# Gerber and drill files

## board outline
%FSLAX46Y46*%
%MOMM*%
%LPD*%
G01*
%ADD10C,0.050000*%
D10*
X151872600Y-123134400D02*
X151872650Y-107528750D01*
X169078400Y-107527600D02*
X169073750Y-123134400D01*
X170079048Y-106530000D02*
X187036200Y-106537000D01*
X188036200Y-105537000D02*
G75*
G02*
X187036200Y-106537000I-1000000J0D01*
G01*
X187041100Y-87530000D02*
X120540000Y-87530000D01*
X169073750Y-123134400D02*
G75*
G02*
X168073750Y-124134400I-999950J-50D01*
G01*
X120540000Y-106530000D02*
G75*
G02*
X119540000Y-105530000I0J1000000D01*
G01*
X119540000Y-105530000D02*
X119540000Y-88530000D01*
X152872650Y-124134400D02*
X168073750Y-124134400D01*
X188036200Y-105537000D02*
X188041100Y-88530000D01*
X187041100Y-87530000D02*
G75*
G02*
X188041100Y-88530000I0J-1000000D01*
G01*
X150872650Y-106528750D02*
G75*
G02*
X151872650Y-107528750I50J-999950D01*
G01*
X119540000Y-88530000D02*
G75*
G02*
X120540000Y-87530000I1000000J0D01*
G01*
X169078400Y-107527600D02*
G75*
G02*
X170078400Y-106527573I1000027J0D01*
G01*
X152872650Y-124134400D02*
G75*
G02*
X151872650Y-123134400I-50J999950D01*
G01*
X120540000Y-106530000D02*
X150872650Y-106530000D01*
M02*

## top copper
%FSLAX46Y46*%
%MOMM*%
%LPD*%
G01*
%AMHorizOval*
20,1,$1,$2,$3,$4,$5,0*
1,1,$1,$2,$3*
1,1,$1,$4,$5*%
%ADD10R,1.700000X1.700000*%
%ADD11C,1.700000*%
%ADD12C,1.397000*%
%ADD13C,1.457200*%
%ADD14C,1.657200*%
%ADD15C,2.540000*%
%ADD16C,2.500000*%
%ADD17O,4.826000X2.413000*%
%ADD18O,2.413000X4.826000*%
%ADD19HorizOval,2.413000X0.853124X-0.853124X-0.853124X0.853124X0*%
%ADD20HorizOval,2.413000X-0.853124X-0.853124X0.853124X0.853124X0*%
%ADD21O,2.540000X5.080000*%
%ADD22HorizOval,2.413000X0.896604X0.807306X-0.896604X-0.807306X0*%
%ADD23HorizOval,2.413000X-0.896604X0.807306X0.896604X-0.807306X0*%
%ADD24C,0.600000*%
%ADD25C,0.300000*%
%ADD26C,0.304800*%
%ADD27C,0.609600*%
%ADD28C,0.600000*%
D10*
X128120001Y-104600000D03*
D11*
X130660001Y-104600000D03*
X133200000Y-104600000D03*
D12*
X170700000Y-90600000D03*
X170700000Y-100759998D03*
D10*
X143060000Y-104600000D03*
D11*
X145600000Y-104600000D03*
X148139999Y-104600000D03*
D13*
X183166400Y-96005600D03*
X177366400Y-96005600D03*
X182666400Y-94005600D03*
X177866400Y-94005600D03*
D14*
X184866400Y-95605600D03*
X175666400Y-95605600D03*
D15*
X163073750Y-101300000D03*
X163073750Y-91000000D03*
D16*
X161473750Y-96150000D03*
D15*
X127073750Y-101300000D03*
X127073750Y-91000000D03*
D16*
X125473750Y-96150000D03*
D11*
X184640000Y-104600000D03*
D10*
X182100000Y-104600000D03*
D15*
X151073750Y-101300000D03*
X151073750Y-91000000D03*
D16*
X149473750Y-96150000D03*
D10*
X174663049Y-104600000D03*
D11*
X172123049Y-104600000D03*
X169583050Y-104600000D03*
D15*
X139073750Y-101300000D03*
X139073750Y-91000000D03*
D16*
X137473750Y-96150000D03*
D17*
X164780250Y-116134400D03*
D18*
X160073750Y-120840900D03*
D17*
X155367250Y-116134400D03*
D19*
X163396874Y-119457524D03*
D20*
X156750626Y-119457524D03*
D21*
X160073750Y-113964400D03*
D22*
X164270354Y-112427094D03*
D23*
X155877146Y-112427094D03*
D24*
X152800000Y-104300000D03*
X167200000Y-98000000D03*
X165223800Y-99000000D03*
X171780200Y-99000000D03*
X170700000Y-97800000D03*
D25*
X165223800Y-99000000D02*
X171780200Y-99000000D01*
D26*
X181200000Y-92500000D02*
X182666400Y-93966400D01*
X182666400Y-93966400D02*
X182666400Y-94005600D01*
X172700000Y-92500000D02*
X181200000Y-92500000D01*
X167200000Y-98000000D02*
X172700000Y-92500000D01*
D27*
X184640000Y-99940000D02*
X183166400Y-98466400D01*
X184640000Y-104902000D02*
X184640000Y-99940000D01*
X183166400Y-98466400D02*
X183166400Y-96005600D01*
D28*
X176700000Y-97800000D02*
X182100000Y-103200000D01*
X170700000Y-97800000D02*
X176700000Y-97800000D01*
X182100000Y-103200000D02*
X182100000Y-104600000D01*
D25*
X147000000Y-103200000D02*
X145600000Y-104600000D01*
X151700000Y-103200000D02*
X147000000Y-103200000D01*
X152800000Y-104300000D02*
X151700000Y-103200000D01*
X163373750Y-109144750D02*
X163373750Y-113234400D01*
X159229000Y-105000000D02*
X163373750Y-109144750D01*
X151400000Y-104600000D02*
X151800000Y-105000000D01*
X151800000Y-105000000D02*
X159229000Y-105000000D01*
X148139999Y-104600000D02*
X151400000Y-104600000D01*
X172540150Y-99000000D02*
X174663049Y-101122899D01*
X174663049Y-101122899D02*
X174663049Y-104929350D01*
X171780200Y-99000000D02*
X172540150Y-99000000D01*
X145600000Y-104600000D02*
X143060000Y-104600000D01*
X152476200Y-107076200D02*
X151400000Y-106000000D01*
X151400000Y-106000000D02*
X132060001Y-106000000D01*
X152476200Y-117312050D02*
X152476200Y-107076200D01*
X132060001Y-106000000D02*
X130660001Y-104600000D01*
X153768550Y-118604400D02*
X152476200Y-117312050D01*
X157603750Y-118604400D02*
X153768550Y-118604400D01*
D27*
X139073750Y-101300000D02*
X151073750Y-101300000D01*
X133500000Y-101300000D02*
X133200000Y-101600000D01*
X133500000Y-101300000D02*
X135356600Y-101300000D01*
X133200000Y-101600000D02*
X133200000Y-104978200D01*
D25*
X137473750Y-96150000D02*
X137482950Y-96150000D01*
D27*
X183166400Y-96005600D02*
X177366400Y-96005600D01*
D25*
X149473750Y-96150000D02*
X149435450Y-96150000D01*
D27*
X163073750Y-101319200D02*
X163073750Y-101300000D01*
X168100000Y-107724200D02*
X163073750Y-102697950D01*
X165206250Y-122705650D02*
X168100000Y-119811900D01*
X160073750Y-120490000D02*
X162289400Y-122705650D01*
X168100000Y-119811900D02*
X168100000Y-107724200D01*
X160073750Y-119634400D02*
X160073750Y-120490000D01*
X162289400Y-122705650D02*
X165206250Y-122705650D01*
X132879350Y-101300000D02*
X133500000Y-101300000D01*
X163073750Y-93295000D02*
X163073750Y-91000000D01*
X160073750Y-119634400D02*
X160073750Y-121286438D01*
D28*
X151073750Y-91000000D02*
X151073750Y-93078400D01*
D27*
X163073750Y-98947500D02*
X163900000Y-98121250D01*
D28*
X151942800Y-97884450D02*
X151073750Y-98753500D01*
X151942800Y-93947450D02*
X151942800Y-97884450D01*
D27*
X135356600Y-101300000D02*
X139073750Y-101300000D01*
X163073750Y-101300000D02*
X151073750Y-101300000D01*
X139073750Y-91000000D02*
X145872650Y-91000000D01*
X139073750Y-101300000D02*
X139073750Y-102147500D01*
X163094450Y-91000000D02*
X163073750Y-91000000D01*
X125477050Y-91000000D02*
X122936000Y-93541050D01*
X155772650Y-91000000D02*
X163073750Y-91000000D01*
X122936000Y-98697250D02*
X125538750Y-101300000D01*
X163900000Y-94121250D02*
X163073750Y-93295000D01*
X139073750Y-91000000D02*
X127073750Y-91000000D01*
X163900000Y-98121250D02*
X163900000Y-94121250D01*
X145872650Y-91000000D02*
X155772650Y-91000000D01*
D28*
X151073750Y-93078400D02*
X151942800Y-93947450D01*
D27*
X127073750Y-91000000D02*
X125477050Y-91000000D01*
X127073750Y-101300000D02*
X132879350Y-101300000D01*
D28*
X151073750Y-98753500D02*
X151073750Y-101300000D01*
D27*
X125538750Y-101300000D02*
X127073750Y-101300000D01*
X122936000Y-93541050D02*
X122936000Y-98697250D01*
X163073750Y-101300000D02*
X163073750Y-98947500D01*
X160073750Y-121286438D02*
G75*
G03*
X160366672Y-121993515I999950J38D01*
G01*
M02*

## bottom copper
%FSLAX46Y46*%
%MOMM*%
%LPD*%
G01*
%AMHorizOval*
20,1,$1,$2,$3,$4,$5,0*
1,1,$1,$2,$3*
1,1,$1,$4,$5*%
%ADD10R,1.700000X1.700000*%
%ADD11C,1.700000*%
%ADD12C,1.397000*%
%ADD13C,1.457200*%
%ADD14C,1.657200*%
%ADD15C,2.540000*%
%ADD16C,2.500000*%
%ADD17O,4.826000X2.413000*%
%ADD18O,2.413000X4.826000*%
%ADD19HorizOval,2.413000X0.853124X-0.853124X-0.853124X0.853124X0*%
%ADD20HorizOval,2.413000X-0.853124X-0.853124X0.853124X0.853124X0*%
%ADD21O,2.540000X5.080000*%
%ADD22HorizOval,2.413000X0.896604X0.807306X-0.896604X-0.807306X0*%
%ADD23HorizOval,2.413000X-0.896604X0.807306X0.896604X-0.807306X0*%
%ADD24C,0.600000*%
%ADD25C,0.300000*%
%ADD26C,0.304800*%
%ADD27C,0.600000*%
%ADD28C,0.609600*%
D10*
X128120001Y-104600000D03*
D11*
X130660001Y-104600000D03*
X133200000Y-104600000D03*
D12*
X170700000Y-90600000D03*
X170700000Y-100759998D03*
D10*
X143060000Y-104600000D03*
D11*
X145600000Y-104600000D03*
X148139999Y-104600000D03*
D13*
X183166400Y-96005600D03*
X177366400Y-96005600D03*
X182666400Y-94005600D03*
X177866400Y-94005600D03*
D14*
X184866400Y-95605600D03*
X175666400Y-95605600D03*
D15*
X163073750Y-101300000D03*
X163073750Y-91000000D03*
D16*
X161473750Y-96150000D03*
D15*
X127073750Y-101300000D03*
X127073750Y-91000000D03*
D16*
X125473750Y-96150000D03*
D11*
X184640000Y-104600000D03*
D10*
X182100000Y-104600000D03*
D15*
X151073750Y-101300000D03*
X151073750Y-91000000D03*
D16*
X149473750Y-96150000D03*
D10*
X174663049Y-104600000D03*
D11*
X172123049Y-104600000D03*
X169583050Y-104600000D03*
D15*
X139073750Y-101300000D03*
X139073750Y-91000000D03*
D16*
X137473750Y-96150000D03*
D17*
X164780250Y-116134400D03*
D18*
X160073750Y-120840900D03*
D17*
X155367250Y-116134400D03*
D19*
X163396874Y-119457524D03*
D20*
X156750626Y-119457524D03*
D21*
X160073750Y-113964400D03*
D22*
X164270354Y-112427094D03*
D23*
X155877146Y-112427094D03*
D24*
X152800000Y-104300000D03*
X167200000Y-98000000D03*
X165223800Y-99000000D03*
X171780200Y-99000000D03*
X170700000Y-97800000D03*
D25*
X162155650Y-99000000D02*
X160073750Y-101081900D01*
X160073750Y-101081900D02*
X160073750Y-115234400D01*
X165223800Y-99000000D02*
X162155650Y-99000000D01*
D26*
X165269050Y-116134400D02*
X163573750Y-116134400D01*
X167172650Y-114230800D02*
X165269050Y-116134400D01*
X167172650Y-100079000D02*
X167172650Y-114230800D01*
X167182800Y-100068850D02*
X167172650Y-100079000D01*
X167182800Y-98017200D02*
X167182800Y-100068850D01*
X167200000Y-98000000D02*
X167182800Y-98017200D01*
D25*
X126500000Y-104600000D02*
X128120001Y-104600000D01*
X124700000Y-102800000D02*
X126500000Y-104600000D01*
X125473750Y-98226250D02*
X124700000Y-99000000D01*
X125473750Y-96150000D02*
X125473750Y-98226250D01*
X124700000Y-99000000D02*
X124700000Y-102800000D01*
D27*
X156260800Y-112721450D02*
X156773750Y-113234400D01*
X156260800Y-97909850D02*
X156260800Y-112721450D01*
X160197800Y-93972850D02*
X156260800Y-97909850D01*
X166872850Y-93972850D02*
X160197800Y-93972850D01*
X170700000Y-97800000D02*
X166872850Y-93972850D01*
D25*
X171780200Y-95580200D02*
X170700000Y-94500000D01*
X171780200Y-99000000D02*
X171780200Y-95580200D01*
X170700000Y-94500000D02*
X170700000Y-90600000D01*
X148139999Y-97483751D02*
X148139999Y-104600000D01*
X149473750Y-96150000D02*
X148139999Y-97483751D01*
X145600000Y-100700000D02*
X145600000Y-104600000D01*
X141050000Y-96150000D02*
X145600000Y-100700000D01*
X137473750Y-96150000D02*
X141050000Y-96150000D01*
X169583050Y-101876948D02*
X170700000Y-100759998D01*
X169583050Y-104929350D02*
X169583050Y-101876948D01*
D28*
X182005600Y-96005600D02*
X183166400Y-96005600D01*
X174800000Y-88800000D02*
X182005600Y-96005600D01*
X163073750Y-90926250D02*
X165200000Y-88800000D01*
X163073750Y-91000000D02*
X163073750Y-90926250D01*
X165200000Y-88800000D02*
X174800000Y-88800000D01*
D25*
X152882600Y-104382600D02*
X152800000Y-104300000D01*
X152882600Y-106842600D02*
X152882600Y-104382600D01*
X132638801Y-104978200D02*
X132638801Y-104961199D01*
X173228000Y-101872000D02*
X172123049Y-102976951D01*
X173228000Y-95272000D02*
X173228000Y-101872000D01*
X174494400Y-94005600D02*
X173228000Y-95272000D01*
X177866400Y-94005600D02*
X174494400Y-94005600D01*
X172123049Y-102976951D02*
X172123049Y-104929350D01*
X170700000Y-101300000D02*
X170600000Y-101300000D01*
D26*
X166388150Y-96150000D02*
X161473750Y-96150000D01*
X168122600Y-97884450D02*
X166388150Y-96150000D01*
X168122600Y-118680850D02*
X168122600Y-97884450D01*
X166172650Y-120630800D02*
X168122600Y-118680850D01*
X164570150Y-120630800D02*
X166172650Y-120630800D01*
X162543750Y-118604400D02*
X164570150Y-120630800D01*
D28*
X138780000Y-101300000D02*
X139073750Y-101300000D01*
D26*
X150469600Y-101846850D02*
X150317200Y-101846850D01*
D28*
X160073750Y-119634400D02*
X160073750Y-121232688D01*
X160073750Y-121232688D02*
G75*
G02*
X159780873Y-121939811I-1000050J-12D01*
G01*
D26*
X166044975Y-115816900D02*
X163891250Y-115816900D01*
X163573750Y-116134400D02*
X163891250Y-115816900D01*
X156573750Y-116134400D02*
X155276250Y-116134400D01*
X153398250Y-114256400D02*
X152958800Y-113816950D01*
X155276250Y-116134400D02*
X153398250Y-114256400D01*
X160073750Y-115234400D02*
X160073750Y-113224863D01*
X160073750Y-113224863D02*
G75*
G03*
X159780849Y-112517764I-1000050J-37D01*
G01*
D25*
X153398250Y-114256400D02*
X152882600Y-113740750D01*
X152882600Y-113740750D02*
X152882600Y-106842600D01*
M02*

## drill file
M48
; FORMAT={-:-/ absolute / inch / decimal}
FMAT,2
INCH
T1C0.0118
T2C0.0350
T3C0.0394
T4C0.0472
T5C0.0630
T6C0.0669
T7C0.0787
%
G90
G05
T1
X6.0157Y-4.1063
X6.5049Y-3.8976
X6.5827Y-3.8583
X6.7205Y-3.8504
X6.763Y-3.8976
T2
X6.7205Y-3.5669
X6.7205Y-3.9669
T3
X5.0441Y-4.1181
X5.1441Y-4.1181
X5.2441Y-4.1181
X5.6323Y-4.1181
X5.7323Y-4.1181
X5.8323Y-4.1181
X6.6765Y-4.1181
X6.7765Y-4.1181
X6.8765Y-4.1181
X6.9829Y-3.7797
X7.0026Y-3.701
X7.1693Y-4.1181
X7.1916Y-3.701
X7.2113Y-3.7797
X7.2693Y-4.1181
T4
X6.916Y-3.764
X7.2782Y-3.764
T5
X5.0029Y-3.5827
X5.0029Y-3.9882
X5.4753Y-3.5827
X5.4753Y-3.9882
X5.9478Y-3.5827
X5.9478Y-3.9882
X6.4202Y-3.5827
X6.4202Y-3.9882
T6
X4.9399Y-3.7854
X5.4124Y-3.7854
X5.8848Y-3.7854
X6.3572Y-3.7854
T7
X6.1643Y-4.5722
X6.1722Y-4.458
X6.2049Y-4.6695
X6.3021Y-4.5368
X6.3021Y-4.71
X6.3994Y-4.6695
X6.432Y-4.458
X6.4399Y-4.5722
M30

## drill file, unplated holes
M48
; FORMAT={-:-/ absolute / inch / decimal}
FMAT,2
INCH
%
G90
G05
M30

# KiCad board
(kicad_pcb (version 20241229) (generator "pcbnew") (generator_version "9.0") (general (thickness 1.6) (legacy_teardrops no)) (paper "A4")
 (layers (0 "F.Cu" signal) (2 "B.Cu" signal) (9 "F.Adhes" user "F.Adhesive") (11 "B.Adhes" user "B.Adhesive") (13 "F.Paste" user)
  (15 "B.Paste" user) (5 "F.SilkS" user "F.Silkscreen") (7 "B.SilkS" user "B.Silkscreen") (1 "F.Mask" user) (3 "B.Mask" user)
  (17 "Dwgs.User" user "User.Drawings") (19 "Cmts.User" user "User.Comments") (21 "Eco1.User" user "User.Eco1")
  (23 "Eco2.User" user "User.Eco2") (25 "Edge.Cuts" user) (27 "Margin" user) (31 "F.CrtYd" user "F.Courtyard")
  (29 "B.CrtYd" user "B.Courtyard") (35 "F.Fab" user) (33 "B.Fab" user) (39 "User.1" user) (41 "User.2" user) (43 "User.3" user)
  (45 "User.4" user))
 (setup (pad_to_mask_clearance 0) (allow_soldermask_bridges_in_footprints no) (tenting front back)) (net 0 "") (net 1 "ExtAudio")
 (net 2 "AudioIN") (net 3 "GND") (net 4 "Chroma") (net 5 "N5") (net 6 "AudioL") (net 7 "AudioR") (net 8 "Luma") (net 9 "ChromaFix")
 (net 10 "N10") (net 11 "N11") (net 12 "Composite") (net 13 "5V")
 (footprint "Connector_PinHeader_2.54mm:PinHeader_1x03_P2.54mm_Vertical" (layer "F.Cu") (at 128.120001 104.6 90)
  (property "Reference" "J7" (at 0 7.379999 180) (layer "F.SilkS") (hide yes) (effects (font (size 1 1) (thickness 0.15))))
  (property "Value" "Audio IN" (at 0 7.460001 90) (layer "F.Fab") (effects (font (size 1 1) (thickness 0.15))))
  (pad "1" thru_hole rect (at 0 0 90) (size 1.7 1.7) (drill 1) (layers "*.Cu" "*.Mask") (remove_unused_layers no) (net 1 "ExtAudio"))
  (pad "2" thru_hole circle (at 0 2.54 90) (size 1.7 1.7) (drill 1) (layers "*.Cu" "*.Mask") (remove_unused_layers no) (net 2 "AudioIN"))
  (pad "3" thru_hole circle (at 0 5.079999 90) (size 1.7 1.7) (drill 1) (layers "*.Cu" "*.Mask") (remove_unused_layers no) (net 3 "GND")))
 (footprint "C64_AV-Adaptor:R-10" (layer "F.Cu") (at 170.7 95.679999 -90)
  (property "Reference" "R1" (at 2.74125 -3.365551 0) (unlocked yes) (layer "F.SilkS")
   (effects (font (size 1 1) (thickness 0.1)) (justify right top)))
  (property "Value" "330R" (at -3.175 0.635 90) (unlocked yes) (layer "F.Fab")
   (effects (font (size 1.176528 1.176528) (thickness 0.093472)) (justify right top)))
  (pad "1" thru_hole circle (at -5.079999 0 270) (size 1.397 1.397) (drill 0.889) (layers "*.Cu" "*.Mask") (remove_unused_layers no)
   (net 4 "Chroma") (solder_mask_margin 0.1016) (thermal_bridge_angle 0))
  (pad "2" thru_hole circle (at 5.079999 0 270) (size 1.397 1.397) (drill 0.889) (layers "*.Cu" "*.Mask") (remove_unused_layers no)
   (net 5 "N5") (solder_mask_margin 0.1016) (thermal_bridge_angle 0)))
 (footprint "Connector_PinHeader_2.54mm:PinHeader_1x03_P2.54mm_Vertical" (layer "F.Cu") (at 143.06 104.6 90)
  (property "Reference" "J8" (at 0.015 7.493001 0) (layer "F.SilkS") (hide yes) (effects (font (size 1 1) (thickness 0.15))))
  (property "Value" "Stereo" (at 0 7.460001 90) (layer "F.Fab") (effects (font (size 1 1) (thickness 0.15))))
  (pad "1" thru_hole rect (at 0 0 90) (size 1.7 1.7) (drill 1) (layers "*.Cu" "*.Mask") (remove_unused_layers no) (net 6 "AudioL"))
  (pad "2" thru_hole circle (at 0 2.54 90) (size 1.7 1.7) (drill 1) (layers "*.Cu" "*.Mask") (remove_unused_layers no) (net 6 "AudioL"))
  (pad "3" thru_hole circle (at 0 5.079999 90) (size 1.7 1.7) (drill 1) (layers "*.Cu" "*.Mask") (remove_unused_layers no) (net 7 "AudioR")))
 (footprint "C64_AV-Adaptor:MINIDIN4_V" (layer "F.Cu") (at 180.2664 95.6056)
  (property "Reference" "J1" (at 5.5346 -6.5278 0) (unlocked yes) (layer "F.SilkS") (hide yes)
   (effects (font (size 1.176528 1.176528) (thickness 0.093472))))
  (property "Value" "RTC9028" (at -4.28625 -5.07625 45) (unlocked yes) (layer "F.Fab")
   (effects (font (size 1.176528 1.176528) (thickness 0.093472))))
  (pad "1" thru_hole circle (at 2.9 0.4) (size 1.4572 1.4572) (drill 1) (layers "*.Cu" "*.Mask") (remove_unused_layers no) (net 3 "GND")
   (solder_mask_margin 0.1016) (thermal_bridge_angle 0))
  (pad "2" thru_hole circle (at -2.9 0.4) (size 1.4572 1.4572) (drill 1) (layers "*.Cu" "*.Mask") (remove_unused_layers no) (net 3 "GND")
   (solder_mask_margin 0.1016) (thermal_bridge_angle 0))
  (pad "3" thru_hole circle (at 2.4 -1.6) (size 1.4572 1.4572) (drill 1) (layers "*.Cu" "*.Mask") (remove_unused_layers no) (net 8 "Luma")
   (solder_mask_margin 0.1016) (thermal_bridge_angle 0))
  (pad "4" thru_hole circle (at -2.4 -1.6) (size 1.4572 1.4572) (drill 1) (layers "*.Cu" "*.Mask") (remove_unused_layers no)
   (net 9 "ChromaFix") (solder_mask_margin 0.1016) (thermal_bridge_angle 0))
  (pad "CS1" thru_hole circle (at 4.6 0) (size 1.6572 1.6572) (drill 1.2) (layers "*.Cu" "*.Mask") (remove_unused_layers no) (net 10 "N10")
   (solder_mask_margin 0.1016) (thermal_bridge_angle 0))
  (pad "CS2" thru_hole circle (at -4.6 0) (size 1.6572 1.6572) (drill 1.2) (layers "*.Cu" "*.Mask") (remove_unused_layers no) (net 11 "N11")
   (solder_mask_margin 0.1016) (thermal_bridge_angle 0)))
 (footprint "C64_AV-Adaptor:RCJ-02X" (layer "F.Cu") (at 163.07375 96.15 90)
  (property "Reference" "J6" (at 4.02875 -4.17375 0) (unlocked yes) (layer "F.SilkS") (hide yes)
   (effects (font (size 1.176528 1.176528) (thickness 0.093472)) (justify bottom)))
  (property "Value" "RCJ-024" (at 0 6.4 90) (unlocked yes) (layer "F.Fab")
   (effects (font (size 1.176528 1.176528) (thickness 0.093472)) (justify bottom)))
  (pad "R1" thru_hole circle (at -5.15 0 90) (size 2.54 2.54) (drill 1.6) (layers "*.Cu" "*.Mask") (remove_unused_layers no) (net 3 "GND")
   (solder_mask_margin 0.1016) (thermal_bridge_angle 0))
  (pad "R2" thru_hole circle (at 5.15 0 90) (size 2.54 2.54) (drill 1.6) (layers "*.Cu" "*.Mask") (remove_unused_layers no) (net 3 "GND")
   (solder_mask_margin 0.1016) (thermal_bridge_angle 0))
  (pad "T" thru_hole circle (at 0 -1.6 90) (size 2.5 2.5) (drill 1.7) (layers "*.Cu" "*.Mask") (remove_unused_layers no)
   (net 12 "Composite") (solder_mask_margin 0.1016) (thermal_bridge_angle 0)))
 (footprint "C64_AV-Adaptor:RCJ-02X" (layer "F.Cu") (at 127.07375 96.15 90)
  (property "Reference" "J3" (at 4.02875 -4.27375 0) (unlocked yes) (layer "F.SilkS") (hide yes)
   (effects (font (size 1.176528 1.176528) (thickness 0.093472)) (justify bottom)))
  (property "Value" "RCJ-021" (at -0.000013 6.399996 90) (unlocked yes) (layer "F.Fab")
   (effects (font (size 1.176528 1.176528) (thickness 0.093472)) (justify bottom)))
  (pad "R1" thru_hole circle (at -5.15 0 90) (size 2.54 2.54) (drill 1.6) (layers "*.Cu" "*.Mask") (remove_unused_layers no) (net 3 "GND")
   (solder_mask_margin 0.1016) (thermal_bridge_angle 0))
  (pad "R2" thru_hole circle (at 5.15 0 90) (size 2.54 2.54) (drill 1.6) (layers "*.Cu" "*.Mask") (remove_unused_layers no) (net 3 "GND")
   (solder_mask_margin 0.1016) (thermal_bridge_angle 0))
  (pad "T" thru_hole circle (at 0 -1.6 90) (size 2.5 2.5) (drill 1.7) (layers "*.Cu" "*.Mask") (remove_unused_layers no) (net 1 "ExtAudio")
   (solder_mask_margin 0.1016) (thermal_bridge_angle 0)))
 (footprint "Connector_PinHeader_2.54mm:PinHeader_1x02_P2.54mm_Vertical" (layer "F.Cu") (at 182.1 104.6 90)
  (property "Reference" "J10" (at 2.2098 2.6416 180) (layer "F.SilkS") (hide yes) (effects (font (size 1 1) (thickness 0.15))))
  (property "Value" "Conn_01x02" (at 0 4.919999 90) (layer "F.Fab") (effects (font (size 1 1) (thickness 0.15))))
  (pad "1" thru_hole rect (at 0 0 90) (size 1.7 1.7) (drill 1) (layers "*.Cu" "*.Mask") (remove_unused_layers no) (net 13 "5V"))
  (pad "2" thru_hole circle (at 0 2.54 90) (size 1.7 1.7) (drill 1) (layers "*.Cu" "*.Mask") (remove_unused_layers no) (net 3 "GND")))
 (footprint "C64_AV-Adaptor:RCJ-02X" (layer "F.Cu") (at 151.07375 96.15 90)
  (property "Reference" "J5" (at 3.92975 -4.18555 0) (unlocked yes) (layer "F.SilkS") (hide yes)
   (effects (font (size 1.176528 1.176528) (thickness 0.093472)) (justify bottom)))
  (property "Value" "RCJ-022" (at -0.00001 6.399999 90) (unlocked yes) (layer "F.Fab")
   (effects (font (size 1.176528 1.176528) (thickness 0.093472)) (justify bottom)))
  (pad "R1" thru_hole circle (at -5.15 0 90) (size 2.54 2.54) (drill 1.6) (layers "*.Cu" "*.Mask") (remove_unused_layers no) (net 3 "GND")
   (solder_mask_margin 0.1016) (thermal_bridge_angle 0))
  (pad "R2" thru_hole circle (at 5.15 0 90) (size 2.54 2.54) (drill 1.6) (layers "*.Cu" "*.Mask") (remove_unused_layers no) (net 3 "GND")
   (solder_mask_margin 0.1016) (thermal_bridge_angle 0))
  (pad "T" thru_hole circle (at 0 -1.6 90) (size 2.5 2.5) (drill 1.7) (layers "*.Cu" "*.Mask") (remove_unused_layers no) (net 7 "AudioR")
   (solder_mask_margin 0.1016) (thermal_bridge_angle 0)))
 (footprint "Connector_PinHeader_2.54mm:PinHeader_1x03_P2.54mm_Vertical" (layer "F.Cu") (at 174.663049 104.6 -90)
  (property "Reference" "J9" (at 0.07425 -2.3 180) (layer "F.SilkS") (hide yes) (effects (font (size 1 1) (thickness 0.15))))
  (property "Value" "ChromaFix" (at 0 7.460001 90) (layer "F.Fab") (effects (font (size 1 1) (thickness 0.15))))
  (pad "1" thru_hole rect (at 0 0 270) (size 1.7 1.7) (drill 1) (layers "*.Cu" "*.Mask") (remove_unused_layers no) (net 4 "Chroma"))
  (pad "2" thru_hole circle (at 0 2.54 270) (size 1.7 1.7) (drill 1) (layers "*.Cu" "*.Mask") (remove_unused_layers no) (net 9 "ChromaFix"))
  (pad "3" thru_hole circle (at 0 5.079999 270) (size 1.7 1.7) (drill 1) (layers "*.Cu" "*.Mask") (remove_unused_layers no) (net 5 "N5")))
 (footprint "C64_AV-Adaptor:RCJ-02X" (layer "F.Cu") (at 139.07375 96.15 90)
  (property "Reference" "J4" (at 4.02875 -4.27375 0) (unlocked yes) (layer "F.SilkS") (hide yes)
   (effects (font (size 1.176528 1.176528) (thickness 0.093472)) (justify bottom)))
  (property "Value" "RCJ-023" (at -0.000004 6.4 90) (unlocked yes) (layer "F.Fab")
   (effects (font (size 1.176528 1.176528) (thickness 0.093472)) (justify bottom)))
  (pad "R1" thru_hole circle (at -5.15 0 90) (size 2.54 2.54) (drill 1.6) (layers "*.Cu" "*.Mask") (remove_unused_layers no) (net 3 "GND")
   (solder_mask_margin 0.1016) (thermal_bridge_angle 0))
  (pad "R2" thru_hole circle (at 5.15 0 90) (size 2.54 2.54) (drill 1.6) (layers "*.Cu" "*.Mask") (remove_unused_layers no) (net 3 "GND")
   (solder_mask_margin 0.1016) (thermal_bridge_angle 0))
  (pad "T" thru_hole circle (at 0 -1.6 90) (size 2.5 2.5) (drill 1.7) (layers "*.Cu" "*.Mask") (remove_unused_layers no) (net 6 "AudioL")
   (solder_mask_margin 0.1016) (thermal_bridge_angle 0)))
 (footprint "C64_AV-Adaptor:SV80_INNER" (layer "B.Cu") (at 160.07375 116.1344)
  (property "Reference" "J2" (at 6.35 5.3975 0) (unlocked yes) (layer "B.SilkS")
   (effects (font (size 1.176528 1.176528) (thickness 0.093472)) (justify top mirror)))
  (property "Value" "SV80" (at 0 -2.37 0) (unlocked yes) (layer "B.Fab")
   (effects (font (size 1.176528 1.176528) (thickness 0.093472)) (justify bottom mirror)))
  (pad "1" thru_hole oval (at 3.5 0) (size 4.826 2.413) (drill 2 (offset 1.2065 0)) (layers "*.Cu" "*.Mask") (remove_unused_layers no)
   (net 8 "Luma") (solder_mask_margin 0.1016) (thermal_bridge_angle 0))
  (pad "2" thru_hole oval (at 0 3.5 270) (size 4.826 2.413) (drill 2 (offset 1.2065 0)) (layers "*.Cu" "*.Mask") (remove_unused_layers no)
   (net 3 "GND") (solder_mask_margin 0.1016) (thermal_bridge_angle 0))
  (pad "3" thru_hole oval (at -3.5 0 180) (size 4.826 2.413) (drill 2 (offset 1.2065 0)) (layers "*.Cu" "*.Mask") (remove_unused_layers no)
   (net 6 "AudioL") (solder_mask_margin 0.1016) (thermal_bridge_angle 0))
  (pad "4" thru_hole oval (at 2.47 2.47 315) (size 4.826 2.413) (drill 2 (offset 1.2065 0)) (layers "*.Cu" "*.Mask")
   (remove_unused_layers no) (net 12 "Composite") (solder_mask_margin 0.1016) (thermal_bridge_angle 0))
  (pad "5" thru_hole oval (at -2.47 2.47 225) (size 4.826 2.413) (drill 2 (offset 1.2065 0)) (layers "*.Cu" "*.Mask")
   (remove_unused_layers no) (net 2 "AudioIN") (solder_mask_margin 0.1016) (thermal_bridge_angle 0))
  (pad "6" thru_hole oval (at 0 -0.9 90) (size 5.08 2.54) (drill 2 (offset 1.27 0)) (layers "*.Cu" "*.Mask") (remove_unused_layers no)
   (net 4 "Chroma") (solder_mask_margin 0.1016) (thermal_bridge_angle 0))
  (pad "7" thru_hole oval (at 3.3 -2.9 42) (size 4.826 2.413) (drill 2 (offset 1.2065 0)) (layers "*.Cu" "*.Mask") (remove_unused_layers no)
   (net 7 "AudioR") (solder_mask_margin 0.1016) (thermal_bridge_angle 0))
  (pad "8" thru_hole oval (at -3.3 -2.9 138) (size 4.826 2.413) (drill 2 (offset 1.2065 0)) (layers "*.Cu" "*.Mask")
   (remove_unused_layers no) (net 13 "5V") (solder_mask_margin 0.1016) (thermal_bridge_angle 0)))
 (gr_line (start 151.8726 123.1344) (end 151.87265 107.52875) (stroke (width 0.05) (type default)) (layer "Edge.Cuts"))
 (gr_line (start 170.079048 106.53) (end 187.0362 106.537) (stroke (width 0.05) (type default)) (layer "Edge.Cuts"))
 (gr_arc (start 188.0362 105.537) (mid 187.743307 106.244107) (end 187.0362 106.537) (stroke (width 0.05) (type solid)) (layer "Edge.Cuts"))
 (gr_line (start 187.0411 87.53) (end 120.54 87.53) (stroke (width 0.05) (type default)) (layer "Edge.Cuts"))
 (gr_arc (start 169.07375 123.1344) (mid 168.780857 123.841507) (end 168.07375 124.1344) (stroke (width 0.05) (type solid))
  (layer "Edge.Cuts"))
 (gr_arc (start 120.54 106.53) (mid 119.832893 106.237107) (end 119.54 105.53) (stroke (width 0.05) (type solid)) (layer "Edge.Cuts"))
 (gr_line (start 119.54 105.53) (end 119.54 88.53) (stroke (width 0.05) (type solid)) (layer "Edge.Cuts"))
 (gr_line (start 152.87265 124.1344) (end 168.07375 124.1344) (stroke (width 0.05) (type default)) (layer "Edge.Cuts"))
 (gr_line (start 188.0362 105.537) (end 188.0411 88.53) (stroke (width 0.05) (type default)) (layer "Edge.Cuts"))
 (gr_arc (start 187.0411 87.53) (mid 187.748207 87.822893) (end 188.0411 88.53) (stroke (width 0.05) (type solid)) (layer "Edge.Cuts"))
 (gr_arc (start 150.87265 106.52875) (mid 151.579757 106.821643) (end 151.87265 107.52875) (stroke (width 0.05) (type solid))
  (layer "Edge.Cuts"))
 (gr_arc (start 119.54 88.53) (mid 119.832893 87.822893) (end 120.54 87.53) (stroke (width 0.05) (type solid)) (layer "Edge.Cuts"))
 (gr_arc (start 169.0784 107.5276) (mid 169.371293 106.820493) (end 170.0784 106.5276) (stroke (width 0.05) (type solid))
  (layer "Edge.Cuts"))
 (gr_arc (start 152.87265 124.1344) (mid 152.165543 123.841507) (end 151.87265 123.1344) (stroke (width 0.05) (type solid))
  (layer "Edge.Cuts"))
 (gr_line (start 169.0784 107.5276) (end 169.07375 123.1344) (stroke (width 0.05) (type default)) (layer "Edge.Cuts"))
 (gr_line (start 120.54 106.53) (end 150.87265 106.53) (stroke (width 0.05) (type solid)) (layer "Edge.Cuts"))
 (segment (start 172.123049 102.976951) (end 172.123049 104.92935) (width 0.3) (layer "B.Cu") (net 9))
 (segment (start 173.228 95.272) (end 173.228 101.872) (width 0.3) (layer "B.Cu") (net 9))
 (segment (start 174.4944 94.0056) (end 173.228 95.272) (width 0.3) (layer "B.Cu") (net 9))
 (segment (start 173.228 101.872) (end 172.123049 102.976951) (width 0.3) (layer "B.Cu") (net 9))
 (segment (start 177.8664 94.0056) (end 174.4944 94.0056) (width 0.3) (layer "B.Cu") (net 9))
 (segment (start 162.2894 122.70565) (end 165.20625 122.70565) (width 0.6096) (layer "F.Cu") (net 3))
 (segment (start 160.07375 120.49) (end 162.2894 122.70565) (width 0.6096) (layer "F.Cu") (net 3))
 (segment (start 163.07375 101.3192) (end 163.07375 101.3) (width 0.6096) (layer "F.Cu") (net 3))
 (segment (start 132.87935 101.3) (end 133.5 101.3) (width 0.6096) (layer "F.Cu") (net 3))
 (segment (start 163.07375 93.295) (end 163.07375 91) (width 0.6096) (layer "F.Cu") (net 3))
 (segment (start 160.07375 119.6344) (end 160.07375 121.286438) (width 0.6096) (layer "F.Cu") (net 3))
 (segment (start 151.07375 91) (end 151.07375 93.0784) (width 0.6) (layer "F.Cu") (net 3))
 (segment (start 163.07375 98.9475) (end 163.9 98.12125) (width 0.6096) (layer "F.Cu") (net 3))
 (segment (start 151.9428 97.88445) (end 151.07375 98.7535) (width 0.6) (layer "F.Cu") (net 3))
 (segment (start 151.9428 93.94745) (end 151.9428 97.88445) (width 0.6) (layer "F.Cu") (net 3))
 (segment (start 133.5 101.3) (end 135.3566 101.3) (width 0.6096) (layer "F.Cu") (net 3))
 (segment (start 135.3566 101.3) (end 139.07375 101.3) (width 0.6096) (layer "F.Cu") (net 3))
 (segment (start 163.07375 101.3) (end 151.07375 101.3) (width 0.6096) (layer "F.Cu") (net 3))
 (segment (start 139.07375 91) (end 145.87265 91) (width 0.6096) (layer "F.Cu") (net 3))
 (segment (start 168.1 107.7242) (end 163.07375 102.69795) (width 0.6096) (layer "F.Cu") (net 3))
 (segment (start 139.07375 101.3) (end 139.07375 102.1475) (width 0.6096) (layer "F.Cu") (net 3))
 (segment (start 163.09445 91) (end 163.07375 91) (width 0.6096) (layer "F.Cu") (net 3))
 (segment (start 125.47705 91) (end 122.936 93.54105) (width 0.6096) (layer "F.Cu") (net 3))
 (segment (start 133.2 101.6) (end 133.2 104.9782) (width 0.6096) (layer "F.Cu") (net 3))
 (segment (start 155.77265 91) (end 163.07375 91) (width 0.6096) (layer "F.Cu") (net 3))
 (segment (start 133.5 101.3) (end 133.2 101.6) (width 0.6096) (layer "F.Cu") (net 3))
 (segment (start 122.936 98.69725) (end 125.53875 101.3) (width 0.6096) (layer "F.Cu") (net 3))
 (segment (start 163.9 94.12125) (end 163.07375 93.295) (width 0.6096) (layer "F.Cu") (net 3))
 (segment (start 139.07375 91) (end 127.07375 91) (width 0.6096) (layer "F.Cu") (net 3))
 (segment (start 163.9 98.12125) (end 163.9 94.12125) (width 0.6096) (layer "F.Cu") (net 3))
 (segment (start 139.07375 101.3) (end 151.07375 101.3) (width 0.6096) (layer "F.Cu") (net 3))
 (segment (start 160.07375 119.6344) (end 160.07375 120.49) (width 0.6096) (layer "F.Cu") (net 3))
 (segment (start 145.87265 91) (end 155.77265 91) (width 0.6096) (layer "F.Cu") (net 3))
 (segment (start 151.07375 93.0784) (end 151.9428 93.94745) (width 0.6) (layer "F.Cu") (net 3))
 (segment (start 127.07375 91) (end 125.47705 91) (width 0.6096) (layer "F.Cu") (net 3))
 (segment (start 127.07375 101.3) (end 132.87935 101.3) (width 0.6096) (layer "F.Cu") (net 3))
 (segment (start 183.1664 98.4664) (end 183.1664 96.0056) (width 0.6096) (layer "F.Cu") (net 3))
 (segment (start 151.07375 98.7535) (end 151.07375 101.3) (width 0.6) (layer "F.Cu") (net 3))
 (segment (start 184.64 99.94) (end 183.1664 98.4664) (width 0.6096) (layer "F.Cu") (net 3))
 (segment (start 183.1664 96.0056) (end 177.3664 96.0056) (width 0.6096) (layer "F.Cu") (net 3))
 (segment (start 165.20625 122.70565) (end 168.1 119.8119) (width 0.6096) (layer "F.Cu") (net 3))
 (segment (start 125.53875 101.3) (end 127.07375 101.3) (width 0.6096) (layer "F.Cu") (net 3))
 (segment (start 184.64 104.902) (end 184.64 99.94) (width 0.6096) (layer "F.Cu") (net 3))
 (segment (start 168.1 119.8119) (end 168.1 107.7242) (width 0.6096) (layer "F.Cu") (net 3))
 (segment (start 122.936 93.54105) (end 122.936 98.69725) (width 0.6096) (layer "F.Cu") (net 3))
 (segment (start 163.07375 101.3) (end 163.07375 98.9475) (width 0.6096) (layer "F.Cu") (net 3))
 (arc (start 160.07375 121.286438) (mid 160.14987 121.669121) (end 160.366643 121.993544) (width 0.6096) (layer "F.Cu") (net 3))
 (segment (start 138.78 101.3) (end 139.07375 101.3) (width 0.6096) (layer "B.Cu") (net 3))
 (segment (start 163.07375 91) (end 163.07375 90.92625) (width 0.6096) (layer "B.Cu") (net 3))
 (segment (start 150.4696 101.84685) (end 150.3172 101.84685) (width 0.3048) (layer "B.Cu") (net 3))
 (segment (start 163.07375 90.92625) (end 165.2 88.8) (width 0.6096) (layer "B.Cu") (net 3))
 (segment (start 160.07375 119.6344) (end 160.07375 121.232688) (width 0.6096) (layer "B.Cu") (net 3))
 (segment (start 182.0056 96.0056) (end 183.1664 96.0056) (width 0.6096) (layer "B.Cu") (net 3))
 (segment (start 165.2 88.8) (end 174.8 88.8) (width 0.6096) (layer "B.Cu") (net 3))
 (segment (start 132.638801 104.9782) (end 132.638801 104.961199) (width 0.3) (layer "B.Cu") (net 3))
 (segment (start 174.8 88.8) (end 182.0056 96.0056) (width 0.6096) (layer "B.Cu") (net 3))
 (arc (start 160.07375 121.232688) (mid 159.997629 121.615371) (end 159.780856 121.939794) (width 0.6096) (layer "B.Cu") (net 3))
 (segment (start 182.6664 93.9664) (end 182.6664 94.0056) (width 0.3048) (layer "F.Cu") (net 8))
 (segment (start 181.2 92.5) (end 182.6664 93.9664) (width 0.3048) (layer "F.Cu") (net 8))
 (segment (start 167.2 98) (end 172.7 92.5) (width 0.3048) (layer "F.Cu") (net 8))
 (segment (start 172.7 92.5) (end 181.2 92.5) (width 0.3048) (layer "F.Cu") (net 8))
 (via (at 167.2 98) (size 0.6) (drill 0.3) (layers "F.Cu" "B.Cu") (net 8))
 (segment (start 167.17265 114.2308) (end 165.26905 116.1344) (width 0.3048) (layer "B.Cu") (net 8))
 (segment (start 165.26905 116.1344) (end 163.57375 116.1344) (width 0.3048) (layer "B.Cu") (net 8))
 (segment (start 167.1828 98.0172) (end 167.1828 100.06885) (width 0.3048) (layer "B.Cu") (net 8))
 (segment (start 167.1828 100.06885) (end 167.17265 100.079) (width 0.3048) (layer "B.Cu") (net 8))
 (segment (start 166.044975 115.8169) (end 163.89125 115.8169) (width 0.3048) (layer "B.Cu") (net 8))
 (segment (start 167.2 98) (end 167.1828 98.0172) (width 0.3048) (layer "B.Cu") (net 8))
 (segment (start 163.57375 116.1344) (end 163.89125 115.8169) (width 0.3048) (layer "B.Cu") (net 8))
 (segment (start 167.17265 100.079) (end 167.17265 114.2308) (width 0.3048) (layer "B.Cu") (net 8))
 (segment (start 168.1226 118.68085) (end 168.1226 97.88445) (width 0.3048) (layer "B.Cu") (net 12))
 (segment (start 168.1226 97.88445) (end 166.38815 96.15) (width 0.3048) (layer "B.Cu") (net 12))
 (segment (start 166.17265 120.6308) (end 168.1226 118.68085) (width 0.3048) (layer "B.Cu") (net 12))
 (segment (start 166.38815 96.15) (end 161.47375 96.15) (width 0.3048) (layer "B.Cu") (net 12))
 (segment (start 162.54375 118.6044) (end 164.57015 120.6308) (width 0.3048) (layer "B.Cu") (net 12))
 (segment (start 164.57015 120.6308) (end 166.17265 120.6308) (width 0.3048) (layer "B.Cu") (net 12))
 (segment (start 151.8 105) (end 159.229 105) (width 0.3) (layer "F.Cu") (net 7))
 (segment (start 149.47375 96.15) (end 149.43545 96.15) (width 0.3) (layer "F.Cu") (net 7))
 (segment (start 151.4 104.6) (end 151.8 105) (width 0.3) (layer "F.Cu") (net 7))
 (segment (start 148.139999 104.6) (end 151.4 104.6) (width 0.3) (layer "F.Cu") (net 7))
 (segment (start 163.37375 109.14475) (end 163.37375 113.2344) (width 0.3) (layer "F.Cu") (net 7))
 (segment (start 159.229 105) (end 163.37375 109.14475) (width 0.3) (layer "F.Cu") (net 7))
 (segment (start 148.139999 97.483751) (end 148.139999 104.6) (width 0.3) (layer "B.Cu") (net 7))
 (segment (start 149.47375 96.15) (end 148.139999 97.483751) (width 0.3) (layer "B.Cu") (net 7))
 (segment (start 151.7 103.2) (end 147 103.2) (width 0.3) (layer "F.Cu") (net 6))
 (segment (start 147 103.2) (end 145.6 104.6) (width 0.3) (layer "F.Cu") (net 6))
 (segment (start 145.6 104.6) (end 143.06 104.6) (width 0.3) (layer "F.Cu") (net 6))
 (segment (start 152.8 104.3) (end 151.7 103.2) (width 0.3) (layer "F.Cu") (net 6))
 (segment (start 137.47375 96.15) (end 137.48295 96.15) (width 0.3) (layer "F.Cu") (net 6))
 (via (at 152.8 104.3) (size 0.6) (drill 0.3) (layers "F.Cu" "B.Cu") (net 6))
 (segment (start 153.39825 114.2564) (end 152.8826 113.74075) (width 0.3) (layer "B.Cu") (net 6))
 (segment (start 156.57375 116.1344) (end 155.27625 116.1344) (width 0.3048) (layer "B.Cu") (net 6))
 (segment (start 137.47375 96.15) (end 141.05 96.15) (width 0.3) (layer "B.Cu") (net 6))
 (segment (start 153.39825 114.2564) (end 152.9588 113.81695) (width 0.3048) (layer "B.Cu") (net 6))
 (segment (start 141.05 96.15) (end 145.6 100.7) (width 0.3) (layer "B.Cu") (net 6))
 (segment (start 145.6 100.7) (end 145.6 104.6) (width 0.3) (layer "B.Cu") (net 6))
 (segment (start 152.8826 106.8426) (end 152.8826 104.3826) (width 0.3) (layer "B.Cu") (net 6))
 (segment (start 152.8826 113.74075) (end 152.8826 106.8426) (width 0.3) (layer "B.Cu") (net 6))
 (segment (start 155.27625 116.1344) (end 153.39825 114.2564) (width 0.3048) (layer "B.Cu") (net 6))
 (segment (start 152.8826 104.3826) (end 152.8 104.3) (width 0.3) (layer "B.Cu") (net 6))
 (segment (start 174.663049 101.122899) (end 174.663049 104.92935) (width 0.3) (layer "F.Cu") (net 4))
 (segment (start 165.2238 99) (end 171.7802 99) (width 0.3) (layer "F.Cu") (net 4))
 (segment (start 171.7802 99) (end 172.54015 99) (width 0.3) (layer "F.Cu") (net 4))
 (segment (start 172.54015 99) (end 174.663049 101.122899) (width 0.3) (layer "F.Cu") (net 4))
 (via (at 165.2238 99) (size 0.6) (drill 0.3) (layers "F.Cu" "B.Cu") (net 4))
 (via (at 171.7802 99) (size 0.6) (drill 0.3) (layers "F.Cu" "B.Cu") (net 4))
 (segment (start 165.2238 99) (end 162.15565 99) (width 0.3) (layer "B.Cu") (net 4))
 (segment (start 171.7802 95.5802) (end 170.7 94.5) (width 0.3) (layer "B.Cu") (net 4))
 (segment (start 160.07375 101.0819) (end 160.07375 115.2344) (width 0.3) (layer "B.Cu") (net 4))
 (segment (start 171.7802 99) (end 171.7802 95.5802) (width 0.3) (layer "B.Cu") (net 4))
 (segment (start 162.15565 99) (end 160.07375 101.0819) (width 0.3) (layer "B.Cu") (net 4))
 (segment (start 160.07375 115.2344) (end 160.07375 113.224863) (width 0.3048) (layer "B.Cu") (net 4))
 (segment (start 170.7 94.5) (end 170.7 90.6) (width 0.3) (layer "B.Cu") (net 4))
 (arc (start 160.07375 113.224863) (mid 159.997629 112.84218) (end 159.780856 112.517757) (width 0.3048) (layer "B.Cu") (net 4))
 (segment (start 182.1 103.2) (end 182.1 104.6) (width 0.6) (layer "F.Cu") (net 13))
 (segment (start 170.7 97.8) (end 176.7 97.8) (width 0.6) (layer "F.Cu") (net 13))
 (segment (start 176.7 97.8) (end 182.1 103.2) (width 0.6) (layer "F.Cu") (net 13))
 (via (at 170.7 97.8) (size 0.6) (drill 0.3) (layers "F.Cu" "B.Cu") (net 13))
 (segment (start 160.1978 93.97285) (end 156.2608 97.90985) (width 0.6) (layer "B.Cu") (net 13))
 (segment (start 170.7 97.8) (end 166.87285 93.97285) (width 0.6) (layer "B.Cu") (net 13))
 (segment (start 156.2608 112.72145) (end 156.77375 113.2344) (width 0.6) (layer "B.Cu") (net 13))
 (segment (start 166.87285 93.97285) (end 160.1978 93.97285) (width 0.6) (layer "B.Cu") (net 13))
 (segment (start 156.2608 97.90985) (end 156.2608 112.72145) (width 0.6) (layer "B.Cu") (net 13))
 (segment (start 152.4762 107.0762) (end 151.4 106) (width 0.3) (layer "F.Cu") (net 2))
 (segment (start 152.4762 117.31205) (end 152.4762 107.0762) (width 0.3) (layer "F.Cu") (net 2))
 (segment (start 157.60375 118.6044) (end 153.76855 118.6044) (width 0.3) (layer "F.Cu") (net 2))
 (segment (start 151.4 106) (end 132.060001 106) (width 0.3) (layer "F.Cu") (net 2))
 (segment (start 153.76855 118.6044) (end 152.4762 117.31205) (width 0.3) (layer "F.Cu") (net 2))
 (segment (start 132.060001 106) (end 130.660001 104.6) (width 0.3) (layer "F.Cu") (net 2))
 (segment (start 124.7 99) (end 124.7 102.8) (width 0.3) (layer "B.Cu") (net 1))
 (segment (start 124.7 102.8) (end 126.5 104.6) (width 0.3) (layer "B.Cu") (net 1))
 (segment (start 125.47375 98.22625) (end 124.7 99) (width 0.3) (layer "B.Cu") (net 1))
 (segment (start 125.47375 96.15) (end 125.47375 98.22625) (width 0.3) (layer "B.Cu") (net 1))
 (segment (start 126.5 104.6) (end 128.120001 104.6) (width 0.3) (layer "B.Cu") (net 1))
 (segment (start 170.7 101.3) (end 170.6 101.3) (width 0.3) (layer "B.Cu") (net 5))
 (segment (start 169.58305 104.92935) (end 169.58305 101.876948) (width 0.3) (layer "B.Cu") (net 5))
 (segment (start 169.58305 101.876948) (end 170.7 100.759998) (width 0.3) (layer "B.Cu") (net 5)))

